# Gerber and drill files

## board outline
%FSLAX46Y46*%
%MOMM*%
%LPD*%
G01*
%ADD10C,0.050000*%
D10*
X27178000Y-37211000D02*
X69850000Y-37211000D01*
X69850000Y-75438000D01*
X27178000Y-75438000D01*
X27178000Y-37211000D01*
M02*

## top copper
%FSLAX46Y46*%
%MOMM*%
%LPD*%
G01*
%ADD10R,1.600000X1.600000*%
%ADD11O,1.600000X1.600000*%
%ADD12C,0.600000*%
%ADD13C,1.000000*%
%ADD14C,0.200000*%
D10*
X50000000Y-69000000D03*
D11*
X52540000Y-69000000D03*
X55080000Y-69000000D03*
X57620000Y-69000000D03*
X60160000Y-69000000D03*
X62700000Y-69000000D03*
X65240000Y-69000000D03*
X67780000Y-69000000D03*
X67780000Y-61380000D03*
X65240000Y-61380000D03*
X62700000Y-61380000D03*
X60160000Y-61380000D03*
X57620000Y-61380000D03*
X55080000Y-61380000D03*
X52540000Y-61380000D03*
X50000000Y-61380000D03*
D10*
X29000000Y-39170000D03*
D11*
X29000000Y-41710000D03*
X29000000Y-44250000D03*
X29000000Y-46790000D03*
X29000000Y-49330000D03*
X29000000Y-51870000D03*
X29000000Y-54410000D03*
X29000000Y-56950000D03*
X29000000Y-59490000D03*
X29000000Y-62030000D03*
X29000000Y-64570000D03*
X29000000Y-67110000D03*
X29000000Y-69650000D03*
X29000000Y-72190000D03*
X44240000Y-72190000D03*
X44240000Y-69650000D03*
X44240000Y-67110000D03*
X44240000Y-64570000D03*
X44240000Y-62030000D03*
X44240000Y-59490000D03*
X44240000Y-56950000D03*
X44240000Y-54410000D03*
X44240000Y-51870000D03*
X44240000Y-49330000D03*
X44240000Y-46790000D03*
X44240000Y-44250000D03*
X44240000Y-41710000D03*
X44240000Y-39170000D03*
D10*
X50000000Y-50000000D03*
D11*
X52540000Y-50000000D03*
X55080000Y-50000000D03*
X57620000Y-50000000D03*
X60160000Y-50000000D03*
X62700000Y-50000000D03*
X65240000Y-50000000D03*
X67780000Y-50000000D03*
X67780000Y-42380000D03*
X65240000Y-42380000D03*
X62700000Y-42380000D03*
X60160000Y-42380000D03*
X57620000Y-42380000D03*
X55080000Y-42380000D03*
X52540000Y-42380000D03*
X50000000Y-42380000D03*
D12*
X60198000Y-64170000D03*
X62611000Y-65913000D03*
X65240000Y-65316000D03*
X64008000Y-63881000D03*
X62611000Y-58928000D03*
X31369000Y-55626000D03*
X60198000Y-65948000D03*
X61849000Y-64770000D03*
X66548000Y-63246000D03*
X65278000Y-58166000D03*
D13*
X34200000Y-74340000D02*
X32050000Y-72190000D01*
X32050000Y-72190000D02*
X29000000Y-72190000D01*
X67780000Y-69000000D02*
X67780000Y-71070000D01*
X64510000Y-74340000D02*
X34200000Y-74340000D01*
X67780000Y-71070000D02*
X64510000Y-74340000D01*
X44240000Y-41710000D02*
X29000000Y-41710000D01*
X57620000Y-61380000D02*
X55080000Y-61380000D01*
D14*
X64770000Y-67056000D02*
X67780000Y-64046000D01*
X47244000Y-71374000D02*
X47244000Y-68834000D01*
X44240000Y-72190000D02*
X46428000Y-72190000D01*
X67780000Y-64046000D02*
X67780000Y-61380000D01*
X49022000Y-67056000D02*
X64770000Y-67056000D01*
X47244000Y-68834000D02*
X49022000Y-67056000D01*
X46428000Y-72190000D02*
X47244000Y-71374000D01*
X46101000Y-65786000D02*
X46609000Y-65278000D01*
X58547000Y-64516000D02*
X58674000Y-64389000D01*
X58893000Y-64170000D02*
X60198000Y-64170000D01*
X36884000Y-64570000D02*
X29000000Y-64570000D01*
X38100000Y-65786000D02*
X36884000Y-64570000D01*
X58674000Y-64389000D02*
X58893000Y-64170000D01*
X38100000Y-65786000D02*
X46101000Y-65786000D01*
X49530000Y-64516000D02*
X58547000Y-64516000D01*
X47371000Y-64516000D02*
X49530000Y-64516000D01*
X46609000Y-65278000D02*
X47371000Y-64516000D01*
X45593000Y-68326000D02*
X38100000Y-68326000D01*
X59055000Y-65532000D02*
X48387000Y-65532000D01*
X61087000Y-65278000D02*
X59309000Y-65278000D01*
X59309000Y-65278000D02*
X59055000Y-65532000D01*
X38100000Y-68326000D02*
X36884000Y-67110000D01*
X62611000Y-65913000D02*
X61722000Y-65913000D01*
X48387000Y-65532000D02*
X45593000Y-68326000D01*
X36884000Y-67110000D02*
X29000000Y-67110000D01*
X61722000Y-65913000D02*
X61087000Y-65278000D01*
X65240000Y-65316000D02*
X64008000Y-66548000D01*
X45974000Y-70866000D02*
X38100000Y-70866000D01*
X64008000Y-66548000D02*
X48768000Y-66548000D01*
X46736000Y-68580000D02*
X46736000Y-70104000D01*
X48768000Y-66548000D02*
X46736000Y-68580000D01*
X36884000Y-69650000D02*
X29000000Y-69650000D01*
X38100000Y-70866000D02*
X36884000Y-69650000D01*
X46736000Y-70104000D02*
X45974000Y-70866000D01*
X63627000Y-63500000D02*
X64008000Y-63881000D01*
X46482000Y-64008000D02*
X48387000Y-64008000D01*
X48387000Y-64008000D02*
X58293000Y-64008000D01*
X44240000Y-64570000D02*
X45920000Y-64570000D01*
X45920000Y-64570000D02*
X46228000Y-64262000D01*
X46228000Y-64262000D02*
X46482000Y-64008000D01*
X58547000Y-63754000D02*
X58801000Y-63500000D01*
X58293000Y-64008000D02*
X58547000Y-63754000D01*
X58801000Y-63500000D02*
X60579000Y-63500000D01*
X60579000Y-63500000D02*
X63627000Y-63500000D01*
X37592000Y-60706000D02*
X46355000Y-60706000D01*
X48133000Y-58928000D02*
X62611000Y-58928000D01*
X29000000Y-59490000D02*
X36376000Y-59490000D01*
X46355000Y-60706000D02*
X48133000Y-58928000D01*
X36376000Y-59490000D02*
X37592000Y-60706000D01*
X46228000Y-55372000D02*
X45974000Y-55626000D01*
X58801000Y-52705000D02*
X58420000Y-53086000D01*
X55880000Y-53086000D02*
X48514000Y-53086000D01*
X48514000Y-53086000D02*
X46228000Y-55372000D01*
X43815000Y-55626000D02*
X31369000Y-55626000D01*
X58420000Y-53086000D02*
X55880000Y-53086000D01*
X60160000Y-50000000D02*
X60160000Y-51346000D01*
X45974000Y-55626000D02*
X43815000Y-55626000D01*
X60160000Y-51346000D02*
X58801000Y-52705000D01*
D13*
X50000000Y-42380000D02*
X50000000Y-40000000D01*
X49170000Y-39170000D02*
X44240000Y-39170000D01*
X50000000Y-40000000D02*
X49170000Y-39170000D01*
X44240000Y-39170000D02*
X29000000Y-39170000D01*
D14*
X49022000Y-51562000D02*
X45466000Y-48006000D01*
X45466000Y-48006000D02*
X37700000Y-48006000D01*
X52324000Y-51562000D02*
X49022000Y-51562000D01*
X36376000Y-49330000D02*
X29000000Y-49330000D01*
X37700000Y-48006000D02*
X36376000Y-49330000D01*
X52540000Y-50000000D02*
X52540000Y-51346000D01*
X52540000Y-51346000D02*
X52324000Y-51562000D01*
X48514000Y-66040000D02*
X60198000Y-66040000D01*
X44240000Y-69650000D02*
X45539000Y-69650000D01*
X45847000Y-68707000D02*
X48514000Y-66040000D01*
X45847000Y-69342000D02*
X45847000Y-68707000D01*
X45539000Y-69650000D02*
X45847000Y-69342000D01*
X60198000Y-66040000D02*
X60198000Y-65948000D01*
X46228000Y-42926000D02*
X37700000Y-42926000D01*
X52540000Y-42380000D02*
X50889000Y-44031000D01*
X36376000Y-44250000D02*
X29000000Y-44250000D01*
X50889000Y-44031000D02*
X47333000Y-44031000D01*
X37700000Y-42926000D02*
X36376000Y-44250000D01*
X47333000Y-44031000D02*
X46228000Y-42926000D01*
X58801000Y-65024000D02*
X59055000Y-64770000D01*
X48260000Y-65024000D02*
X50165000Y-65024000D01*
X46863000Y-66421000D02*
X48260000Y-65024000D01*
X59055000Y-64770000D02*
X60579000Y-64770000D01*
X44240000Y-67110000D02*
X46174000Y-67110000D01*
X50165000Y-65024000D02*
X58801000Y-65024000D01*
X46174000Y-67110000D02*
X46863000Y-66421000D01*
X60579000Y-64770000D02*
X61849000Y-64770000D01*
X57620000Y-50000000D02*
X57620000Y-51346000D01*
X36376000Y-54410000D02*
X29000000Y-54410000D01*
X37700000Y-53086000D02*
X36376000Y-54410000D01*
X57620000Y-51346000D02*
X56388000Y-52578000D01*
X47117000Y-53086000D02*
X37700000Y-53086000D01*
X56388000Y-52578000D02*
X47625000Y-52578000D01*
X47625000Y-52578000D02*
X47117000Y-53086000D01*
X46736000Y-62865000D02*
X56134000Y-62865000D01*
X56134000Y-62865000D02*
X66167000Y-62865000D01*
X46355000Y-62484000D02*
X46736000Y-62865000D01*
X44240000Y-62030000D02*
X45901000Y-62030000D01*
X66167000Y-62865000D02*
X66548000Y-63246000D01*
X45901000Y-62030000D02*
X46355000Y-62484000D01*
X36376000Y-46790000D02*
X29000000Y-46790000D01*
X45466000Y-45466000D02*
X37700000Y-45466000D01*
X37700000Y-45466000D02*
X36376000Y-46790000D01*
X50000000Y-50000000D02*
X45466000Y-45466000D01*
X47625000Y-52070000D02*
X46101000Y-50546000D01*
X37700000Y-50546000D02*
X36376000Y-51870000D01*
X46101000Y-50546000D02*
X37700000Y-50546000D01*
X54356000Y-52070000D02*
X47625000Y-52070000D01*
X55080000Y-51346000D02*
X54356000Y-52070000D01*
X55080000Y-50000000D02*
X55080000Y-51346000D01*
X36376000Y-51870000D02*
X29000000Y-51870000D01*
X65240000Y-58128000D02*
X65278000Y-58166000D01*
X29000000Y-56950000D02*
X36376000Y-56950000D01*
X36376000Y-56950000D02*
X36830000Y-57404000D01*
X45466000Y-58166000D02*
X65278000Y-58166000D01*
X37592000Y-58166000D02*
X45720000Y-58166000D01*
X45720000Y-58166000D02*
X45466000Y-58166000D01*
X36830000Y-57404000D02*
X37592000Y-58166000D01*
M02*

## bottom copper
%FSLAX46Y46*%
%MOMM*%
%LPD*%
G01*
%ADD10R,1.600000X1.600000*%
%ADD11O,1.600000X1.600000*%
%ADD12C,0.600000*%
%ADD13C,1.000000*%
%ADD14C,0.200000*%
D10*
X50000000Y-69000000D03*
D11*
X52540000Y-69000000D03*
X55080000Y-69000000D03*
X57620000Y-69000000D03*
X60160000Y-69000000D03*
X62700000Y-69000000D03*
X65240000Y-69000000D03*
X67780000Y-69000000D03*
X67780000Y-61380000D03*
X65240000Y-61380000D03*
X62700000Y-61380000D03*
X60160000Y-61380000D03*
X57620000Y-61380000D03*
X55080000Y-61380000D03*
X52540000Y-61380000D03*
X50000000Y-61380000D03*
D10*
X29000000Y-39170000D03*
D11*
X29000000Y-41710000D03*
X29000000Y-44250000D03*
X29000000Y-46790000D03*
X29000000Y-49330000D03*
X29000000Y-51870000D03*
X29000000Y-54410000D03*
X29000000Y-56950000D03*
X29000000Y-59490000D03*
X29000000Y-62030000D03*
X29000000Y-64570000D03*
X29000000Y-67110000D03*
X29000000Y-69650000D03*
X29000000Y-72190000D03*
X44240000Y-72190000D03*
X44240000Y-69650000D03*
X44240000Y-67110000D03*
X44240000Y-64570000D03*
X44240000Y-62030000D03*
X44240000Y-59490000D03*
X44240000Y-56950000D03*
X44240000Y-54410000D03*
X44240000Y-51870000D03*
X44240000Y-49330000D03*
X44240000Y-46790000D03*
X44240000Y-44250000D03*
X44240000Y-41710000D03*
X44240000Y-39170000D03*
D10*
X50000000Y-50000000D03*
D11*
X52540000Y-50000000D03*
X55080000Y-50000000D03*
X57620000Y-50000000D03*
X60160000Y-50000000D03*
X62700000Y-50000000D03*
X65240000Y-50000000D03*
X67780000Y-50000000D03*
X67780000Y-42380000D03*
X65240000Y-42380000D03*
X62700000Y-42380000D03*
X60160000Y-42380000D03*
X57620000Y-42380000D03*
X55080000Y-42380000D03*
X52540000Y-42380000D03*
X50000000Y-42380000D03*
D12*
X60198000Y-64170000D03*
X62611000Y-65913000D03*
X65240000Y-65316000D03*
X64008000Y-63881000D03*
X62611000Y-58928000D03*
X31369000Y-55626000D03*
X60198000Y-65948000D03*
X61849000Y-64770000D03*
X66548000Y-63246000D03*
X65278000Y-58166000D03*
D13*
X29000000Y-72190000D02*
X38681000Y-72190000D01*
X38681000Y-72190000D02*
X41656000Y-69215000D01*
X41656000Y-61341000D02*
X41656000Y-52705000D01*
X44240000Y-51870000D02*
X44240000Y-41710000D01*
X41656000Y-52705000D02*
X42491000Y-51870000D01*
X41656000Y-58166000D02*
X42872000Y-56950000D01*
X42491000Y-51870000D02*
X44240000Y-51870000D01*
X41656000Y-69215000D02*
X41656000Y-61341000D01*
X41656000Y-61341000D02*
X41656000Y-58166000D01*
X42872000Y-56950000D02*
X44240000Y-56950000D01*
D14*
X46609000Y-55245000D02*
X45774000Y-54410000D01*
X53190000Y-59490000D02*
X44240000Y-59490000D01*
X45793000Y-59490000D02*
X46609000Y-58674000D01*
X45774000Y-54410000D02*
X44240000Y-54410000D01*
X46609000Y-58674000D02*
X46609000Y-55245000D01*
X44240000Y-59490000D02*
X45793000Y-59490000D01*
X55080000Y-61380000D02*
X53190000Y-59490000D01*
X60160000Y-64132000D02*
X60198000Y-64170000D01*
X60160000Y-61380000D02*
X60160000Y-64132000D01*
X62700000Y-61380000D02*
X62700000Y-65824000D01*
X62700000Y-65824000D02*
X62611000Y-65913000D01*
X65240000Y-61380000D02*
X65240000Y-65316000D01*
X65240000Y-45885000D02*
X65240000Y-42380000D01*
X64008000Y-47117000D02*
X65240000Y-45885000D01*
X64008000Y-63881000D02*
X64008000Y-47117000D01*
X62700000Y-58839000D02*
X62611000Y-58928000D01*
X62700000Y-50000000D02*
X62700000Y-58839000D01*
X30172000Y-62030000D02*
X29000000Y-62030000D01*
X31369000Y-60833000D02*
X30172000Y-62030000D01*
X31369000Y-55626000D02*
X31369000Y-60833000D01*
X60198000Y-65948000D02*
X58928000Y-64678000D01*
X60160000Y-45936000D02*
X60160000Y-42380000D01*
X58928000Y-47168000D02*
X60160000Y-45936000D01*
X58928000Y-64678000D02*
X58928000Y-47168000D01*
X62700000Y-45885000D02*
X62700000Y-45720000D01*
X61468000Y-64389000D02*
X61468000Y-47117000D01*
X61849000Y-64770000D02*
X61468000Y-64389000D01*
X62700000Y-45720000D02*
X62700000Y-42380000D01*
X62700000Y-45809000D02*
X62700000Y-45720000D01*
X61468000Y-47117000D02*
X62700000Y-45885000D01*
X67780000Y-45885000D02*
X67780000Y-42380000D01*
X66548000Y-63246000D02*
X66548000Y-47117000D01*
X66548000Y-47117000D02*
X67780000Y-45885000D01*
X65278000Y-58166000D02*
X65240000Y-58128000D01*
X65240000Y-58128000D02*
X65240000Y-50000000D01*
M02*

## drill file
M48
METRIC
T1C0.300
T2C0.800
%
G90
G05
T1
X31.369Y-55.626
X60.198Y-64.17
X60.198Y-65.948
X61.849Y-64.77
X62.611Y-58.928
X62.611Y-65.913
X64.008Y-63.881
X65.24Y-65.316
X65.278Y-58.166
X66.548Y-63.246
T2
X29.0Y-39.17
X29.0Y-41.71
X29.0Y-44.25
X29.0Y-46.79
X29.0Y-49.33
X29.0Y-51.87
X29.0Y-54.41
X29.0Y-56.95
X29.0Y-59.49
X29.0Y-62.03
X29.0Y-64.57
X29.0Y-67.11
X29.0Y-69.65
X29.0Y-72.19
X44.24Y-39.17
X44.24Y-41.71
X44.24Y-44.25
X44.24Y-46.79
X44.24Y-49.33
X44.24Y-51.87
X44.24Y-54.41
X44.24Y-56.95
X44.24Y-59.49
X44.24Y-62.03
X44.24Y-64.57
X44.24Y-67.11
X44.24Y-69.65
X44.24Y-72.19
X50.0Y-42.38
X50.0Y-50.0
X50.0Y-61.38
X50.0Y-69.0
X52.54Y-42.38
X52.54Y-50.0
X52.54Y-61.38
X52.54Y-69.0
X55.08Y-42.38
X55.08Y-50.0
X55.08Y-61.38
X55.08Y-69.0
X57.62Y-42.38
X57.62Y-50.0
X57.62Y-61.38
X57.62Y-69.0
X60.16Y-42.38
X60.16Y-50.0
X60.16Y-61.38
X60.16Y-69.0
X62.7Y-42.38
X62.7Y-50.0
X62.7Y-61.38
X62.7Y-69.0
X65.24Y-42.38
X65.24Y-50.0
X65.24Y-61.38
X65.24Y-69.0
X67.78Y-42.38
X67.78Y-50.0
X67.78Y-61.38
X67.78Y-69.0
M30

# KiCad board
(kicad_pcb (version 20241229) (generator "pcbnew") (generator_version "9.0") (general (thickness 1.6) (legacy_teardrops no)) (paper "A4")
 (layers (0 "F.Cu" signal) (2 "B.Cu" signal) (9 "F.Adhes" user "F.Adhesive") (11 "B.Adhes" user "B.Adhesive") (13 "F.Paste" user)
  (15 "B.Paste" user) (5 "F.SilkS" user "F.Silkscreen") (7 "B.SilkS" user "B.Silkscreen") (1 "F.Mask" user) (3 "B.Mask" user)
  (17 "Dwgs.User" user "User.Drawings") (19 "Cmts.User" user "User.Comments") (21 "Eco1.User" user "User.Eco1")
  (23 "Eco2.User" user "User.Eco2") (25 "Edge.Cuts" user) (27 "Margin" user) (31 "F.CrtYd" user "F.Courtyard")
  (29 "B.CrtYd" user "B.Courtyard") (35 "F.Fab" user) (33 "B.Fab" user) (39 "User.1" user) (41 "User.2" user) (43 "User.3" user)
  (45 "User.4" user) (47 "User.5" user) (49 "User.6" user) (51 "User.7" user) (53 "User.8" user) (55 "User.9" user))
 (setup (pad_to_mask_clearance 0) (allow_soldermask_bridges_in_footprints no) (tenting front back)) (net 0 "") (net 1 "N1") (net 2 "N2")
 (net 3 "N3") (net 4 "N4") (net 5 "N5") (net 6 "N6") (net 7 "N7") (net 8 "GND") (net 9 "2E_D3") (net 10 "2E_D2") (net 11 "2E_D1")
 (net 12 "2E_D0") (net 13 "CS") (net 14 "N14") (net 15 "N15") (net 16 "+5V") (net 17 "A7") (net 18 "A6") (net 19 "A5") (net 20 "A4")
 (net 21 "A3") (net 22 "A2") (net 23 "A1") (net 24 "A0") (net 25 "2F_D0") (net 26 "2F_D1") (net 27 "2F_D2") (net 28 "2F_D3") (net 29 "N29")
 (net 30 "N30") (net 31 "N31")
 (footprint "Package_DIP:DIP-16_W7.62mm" (layer "F.Cu") (at 50 69 90)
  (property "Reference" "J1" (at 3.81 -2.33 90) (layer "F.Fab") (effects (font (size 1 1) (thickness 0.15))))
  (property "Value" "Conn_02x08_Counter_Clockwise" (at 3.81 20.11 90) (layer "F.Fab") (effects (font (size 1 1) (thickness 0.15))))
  (pad "1" thru_hole rect (at 0 0 90) (size 1.6 1.6) (drill 0.8) (layers "*.Cu" "*.Mask") (remove_unused_layers no) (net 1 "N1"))
  (pad "2" thru_hole oval (at 0 2.54 90) (size 1.6 1.6) (drill 0.8) (layers "*.Cu" "*.Mask") (remove_unused_layers no) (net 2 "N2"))
  (pad "3" thru_hole oval (at 0 5.08 90) (size 1.6 1.6) (drill 0.8) (layers "*.Cu" "*.Mask") (remove_unused_layers no) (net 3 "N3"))
  (pad "4" thru_hole oval (at 0 7.62 90) (size 1.6 1.6) (drill 0.8) (layers "*.Cu" "*.Mask") (remove_unused_layers no) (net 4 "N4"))
  (pad "5" thru_hole oval (at 0 10.16 90) (size 1.6 1.6) (drill 0.8) (layers "*.Cu" "*.Mask") (remove_unused_layers no) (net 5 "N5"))
  (pad "6" thru_hole oval (at 0 12.7 90) (size 1.6 1.6) (drill 0.8) (layers "*.Cu" "*.Mask") (remove_unused_layers no) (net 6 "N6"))
  (pad "7" thru_hole oval (at 0 15.24 90) (size 1.6 1.6) (drill 0.8) (layers "*.Cu" "*.Mask") (remove_unused_layers no) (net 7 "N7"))
  (pad "8" thru_hole oval (at 0 17.78 90) (size 1.6 1.6) (drill 0.8) (layers "*.Cu" "*.Mask") (remove_unused_layers no) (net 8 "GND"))
  (pad "9" thru_hole oval (at 7.62 17.78 90) (size 1.6 1.6) (drill 0.8) (layers "*.Cu" "*.Mask") (remove_unused_layers no) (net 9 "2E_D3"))
  (pad "10" thru_hole oval (at 7.62 15.24 90) (size 1.6 1.6) (drill 0.8) (layers "*.Cu" "*.Mask") (remove_unused_layers no) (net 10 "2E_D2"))
  (pad "11" thru_hole oval (at 7.62 12.7 90) (size 1.6 1.6) (drill 0.8) (layers "*.Cu" "*.Mask") (remove_unused_layers no) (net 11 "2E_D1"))
  (pad "12" thru_hole oval (at 7.62 10.16 90) (size 1.6 1.6) (drill 0.8) (layers "*.Cu" "*.Mask") (remove_unused_layers no) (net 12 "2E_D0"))
  (pad "13" thru_hole oval (at 7.62 7.62 90) (size 1.6 1.6) (drill 0.8) (layers "*.Cu" "*.Mask") (remove_unused_layers no) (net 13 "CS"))
  (pad "14" thru_hole oval (at 7.62 5.08 90) (size 1.6 1.6) (drill 0.8) (layers "*.Cu" "*.Mask") (remove_unused_layers no) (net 13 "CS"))
  (pad "15" thru_hole oval (at 7.62 2.54 90) (size 1.6 1.6) (drill 0.8) (layers "*.Cu" "*.Mask") (remove_unused_layers no) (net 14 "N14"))
  (pad "16" thru_hole oval (at 7.62 0 90) (size 1.6 1.6) (drill 0.8) (layers "*.Cu" "*.Mask") (remove_unused_layers no) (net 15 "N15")))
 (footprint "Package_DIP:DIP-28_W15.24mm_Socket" (layer "F.Cu") (at 29 39.17)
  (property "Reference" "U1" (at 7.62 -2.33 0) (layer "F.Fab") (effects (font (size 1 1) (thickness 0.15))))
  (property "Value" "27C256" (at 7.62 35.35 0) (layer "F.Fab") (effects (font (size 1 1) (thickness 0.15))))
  (pad "1" thru_hole rect (at 0 0) (size 1.6 1.6) (drill 0.8) (layers "*.Cu" "*.Mask") (remove_unused_layers no) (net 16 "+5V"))
  (pad "2" thru_hole oval (at 0 2.54) (size 1.6 1.6) (drill 0.8) (layers "*.Cu" "*.Mask") (remove_unused_layers no) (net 8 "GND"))
  (pad "3" thru_hole oval (at 0 5.08) (size 1.6 1.6) (drill 0.8) (layers "*.Cu" "*.Mask") (remove_unused_layers no) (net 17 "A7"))
  (pad "4" thru_hole oval (at 0 7.62) (size 1.6 1.6) (drill 0.8) (layers "*.Cu" "*.Mask") (remove_unused_layers no) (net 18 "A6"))
  (pad "5" thru_hole oval (at 0 10.16) (size 1.6 1.6) (drill 0.8) (layers "*.Cu" "*.Mask") (remove_unused_layers no) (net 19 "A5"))
  (pad "6" thru_hole oval (at 0 12.7) (size 1.6 1.6) (drill 0.8) (layers "*.Cu" "*.Mask") (remove_unused_layers no) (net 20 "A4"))
  (pad "7" thru_hole oval (at 0 15.24) (size 1.6 1.6) (drill 0.8) (layers "*.Cu" "*.Mask") (remove_unused_layers no) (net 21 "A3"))
  (pad "8" thru_hole oval (at 0 17.78) (size 1.6 1.6) (drill 0.8) (layers "*.Cu" "*.Mask") (remove_unused_layers no) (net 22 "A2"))
  (pad "9" thru_hole oval (at 0 20.32) (size 1.6 1.6) (drill 0.8) (layers "*.Cu" "*.Mask") (remove_unused_layers no) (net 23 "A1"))
  (pad "10" thru_hole oval (at 0 22.86) (size 1.6 1.6) (drill 0.8) (layers "*.Cu" "*.Mask") (remove_unused_layers no) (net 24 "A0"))
  (pad "11" thru_hole oval (at 0 25.4) (size 1.6 1.6) (drill 0.8) (layers "*.Cu" "*.Mask") (remove_unused_layers no) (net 12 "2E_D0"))
  (pad "12" thru_hole oval (at 0 27.94) (size 1.6 1.6) (drill 0.8) (layers "*.Cu" "*.Mask") (remove_unused_layers no) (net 11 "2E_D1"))
  (pad "13" thru_hole oval (at 0 30.48) (size 1.6 1.6) (drill 0.8) (layers "*.Cu" "*.Mask") (remove_unused_layers no) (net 10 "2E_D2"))
  (pad "14" thru_hole oval (at 0 33.02) (size 1.6 1.6) (drill 0.8) (layers "*.Cu" "*.Mask") (remove_unused_layers no) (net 8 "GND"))
  (pad "15" thru_hole oval (at 15.24 33.02) (size 1.6 1.6) (drill 0.8) (layers "*.Cu" "*.Mask") (remove_unused_layers no) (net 9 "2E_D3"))
  (pad "16" thru_hole oval (at 15.24 30.48) (size 1.6 1.6) (drill 0.8) (layers "*.Cu" "*.Mask") (remove_unused_layers no) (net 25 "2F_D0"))
  (pad "17" thru_hole oval (at 15.24 27.94) (size 1.6 1.6) (drill 0.8) (layers "*.Cu" "*.Mask") (remove_unused_layers no) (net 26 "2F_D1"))
  (pad "18" thru_hole oval (at 15.24 25.4) (size 1.6 1.6) (drill 0.8) (layers "*.Cu" "*.Mask") (remove_unused_layers no) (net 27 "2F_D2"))
  (pad "19" thru_hole oval (at 15.24 22.86) (size 1.6 1.6) (drill 0.8) (layers "*.Cu" "*.Mask") (remove_unused_layers no) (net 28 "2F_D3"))
  (pad "20" thru_hole oval (at 15.24 20.32) (size 1.6 1.6) (drill 0.8) (layers "*.Cu" "*.Mask") (remove_unused_layers no) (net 13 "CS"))
  (pad "21" thru_hole oval (at 15.24 17.78) (size 1.6 1.6) (drill 0.8) (layers "*.Cu" "*.Mask") (remove_unused_layers no) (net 8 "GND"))
  (pad "22" thru_hole oval (at 15.24 15.24) (size 1.6 1.6) (drill 0.8) (layers "*.Cu" "*.Mask") (remove_unused_layers no) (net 13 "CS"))
  (pad "23" thru_hole oval (at 15.24 12.7) (size 1.6 1.6) (drill 0.8) (layers "*.Cu" "*.Mask") (remove_unused_layers no) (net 8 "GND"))
  (pad "24" thru_hole oval (at 15.24 10.16) (size 1.6 1.6) (drill 0.8) (layers "*.Cu" "*.Mask") (remove_unused_layers no) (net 8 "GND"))
  (pad "25" thru_hole oval (at 15.24 7.62) (size 1.6 1.6) (drill 0.8) (layers "*.Cu" "*.Mask") (remove_unused_layers no) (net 8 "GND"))
  (pad "26" thru_hole oval (at 15.24 5.08) (size 1.6 1.6) (drill 0.8) (layers "*.Cu" "*.Mask") (remove_unused_layers no) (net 8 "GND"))
  (pad "27" thru_hole oval (at 15.24 2.54) (size 1.6 1.6) (drill 0.8) (layers "*.Cu" "*.Mask") (remove_unused_layers no) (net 8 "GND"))
  (pad "28" thru_hole oval (at 15.24 0) (size 1.6 1.6) (drill 0.8) (layers "*.Cu" "*.Mask") (remove_unused_layers no) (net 16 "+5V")))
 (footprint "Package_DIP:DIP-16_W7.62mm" (layer "F.Cu") (at 50 50 90)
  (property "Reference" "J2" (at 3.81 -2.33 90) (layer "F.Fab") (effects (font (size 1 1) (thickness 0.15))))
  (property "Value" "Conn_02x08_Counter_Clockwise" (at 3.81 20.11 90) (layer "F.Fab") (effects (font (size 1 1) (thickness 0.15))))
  (pad "1" thru_hole rect (at 0 0 90) (size 1.6 1.6) (drill 0.8) (layers "*.Cu" "*.Mask") (remove_unused_layers no) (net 18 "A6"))
  (pad "2" thru_hole oval (at 0 2.54 90) (size 1.6 1.6) (drill 0.8) (layers "*.Cu" "*.Mask") (remove_unused_layers no) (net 19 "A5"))
  (pad "3" thru_hole oval (at 0 5.08 90) (size 1.6 1.6) (drill 0.8) (layers "*.Cu" "*.Mask") (remove_unused_layers no) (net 20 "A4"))
  (pad "4" thru_hole oval (at 0 7.62 90) (size 1.6 1.6) (drill 0.8) (layers "*.Cu" "*.Mask") (remove_unused_layers no) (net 21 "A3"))
  (pad "5" thru_hole oval (at 0 10.16 90) (size 1.6 1.6) (drill 0.8) (layers "*.Cu" "*.Mask") (remove_unused_layers no) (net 24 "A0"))
  (pad "6" thru_hole oval (at 0 12.7 90) (size 1.6 1.6) (drill 0.8) (layers "*.Cu" "*.Mask") (remove_unused_layers no) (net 23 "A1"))
  (pad "7" thru_hole oval (at 0 15.24 90) (size 1.6 1.6) (drill 0.8) (layers "*.Cu" "*.Mask") (remove_unused_layers no) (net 22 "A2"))
  (pad "8" thru_hole oval (at 0 17.78 90) (size 1.6 1.6) (drill 0.8) (layers "*.Cu" "*.Mask") (remove_unused_layers no) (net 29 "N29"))
  (pad "9" thru_hole oval (at 7.62 17.78 90) (size 1.6 1.6) (drill 0.8) (layers "*.Cu" "*.Mask") (remove_unused_layers no) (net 28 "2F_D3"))
  (pad "10" thru_hole oval (at 7.62 15.24 90) (size 1.6 1.6) (drill 0.8) (layers "*.Cu" "*.Mask") (remove_unused_layers no) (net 27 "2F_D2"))
  (pad "11" thru_hole oval (at 7.62 12.7 90) (size 1.6 1.6) (drill 0.8) (layers "*.Cu" "*.Mask") (remove_unused_layers no) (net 26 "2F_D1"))
  (pad "12" thru_hole oval (at 7.62 10.16 90) (size 1.6 1.6) (drill 0.8) (layers "*.Cu" "*.Mask") (remove_unused_layers no) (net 25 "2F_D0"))
  (pad "13" thru_hole oval (at 7.62 7.62 90) (size 1.6 1.6) (drill 0.8) (layers "*.Cu" "*.Mask") (remove_unused_layers no) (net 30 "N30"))
  (pad "14" thru_hole oval (at 7.62 5.08 90) (size 1.6 1.6) (drill 0.8) (layers "*.Cu" "*.Mask") (remove_unused_layers no) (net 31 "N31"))
  (pad "15" thru_hole oval (at 7.62 2.54 90) (size 1.6 1.6) (drill 0.8) (layers "*.Cu" "*.Mask") (remove_unused_layers no) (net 17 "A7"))
  (pad "16" thru_hole oval (at 7.62 0 90) (size 1.6 1.6) (drill 0.8) (layers "*.Cu" "*.Mask") (remove_unused_layers no) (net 16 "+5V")))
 (gr_rect (start 27.178 37.211) (end 69.85 75.438) (stroke (width 0.05) (type default)) (fill no) (layer "Edge.Cuts"))
 (segment (start 34.2 74.34) (end 32.05 72.19) (width 1) (layer "F.Cu") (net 8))
 (segment (start 32.05 72.19) (end 29 72.19) (width 1) (layer "F.Cu") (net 8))
 (segment (start 67.78 69) (end 67.78 71.07) (width 1) (layer "F.Cu") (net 8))
 (segment (start 64.51 74.34) (end 34.2 74.34) (width 1) (layer "F.Cu") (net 8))
 (segment (start 67.78 71.07) (end 64.51 74.34) (width 1) (layer "F.Cu") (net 8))
 (segment (start 44.24 41.71) (end 29 41.71) (width 1) (layer "F.Cu") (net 8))
 (segment (start 29 72.19) (end 38.681 72.19) (width 1) (layer "B.Cu") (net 8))
 (segment (start 38.681 72.19) (end 41.656 69.215) (width 1) (layer "B.Cu") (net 8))
 (segment (start 41.656 61.341) (end 41.656 52.705) (width 1) (layer "B.Cu") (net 8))
 (segment (start 44.24 51.87) (end 44.24 41.71) (width 1) (layer "B.Cu") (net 8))
 (segment (start 41.656 52.705) (end 42.491 51.87) (width 1) (layer "B.Cu") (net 8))
 (segment (start 41.656 58.166) (end 42.872 56.95) (width 1) (layer "B.Cu") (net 8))
 (segment (start 42.491 51.87) (end 44.24 51.87) (width 1) (layer "B.Cu") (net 8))
 (segment (start 41.656 69.215) (end 41.656 61.341) (width 1) (layer "B.Cu") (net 8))
 (segment (start 41.656 61.341) (end 41.656 58.166) (width 1) (layer "B.Cu") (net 8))
 (segment (start 42.872 56.95) (end 44.24 56.95) (width 1) (layer "B.Cu") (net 8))
 (segment (start 57.62 61.38) (end 55.08 61.38) (width 1) (layer "F.Cu") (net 13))
 (segment (start 46.609 55.245) (end 45.774 54.41) (width 0.2) (layer "B.Cu") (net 13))
 (segment (start 53.19 59.49) (end 44.24 59.49) (width 0.2) (layer "B.Cu") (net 13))
 (segment (start 45.793 59.49) (end 46.609 58.674) (width 0.2) (layer "B.Cu") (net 13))
 (segment (start 45.774 54.41) (end 44.24 54.41) (width 0.2) (layer "B.Cu") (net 13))
 (segment (start 46.609 58.674) (end 46.609 55.245) (width 0.2) (layer "B.Cu") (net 13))
 (segment (start 44.24 59.49) (end 45.793 59.49) (width 0.2) (layer "B.Cu") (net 13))
 (segment (start 55.08 61.38) (end 53.19 59.49) (width 0.2) (layer "B.Cu") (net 13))
 (segment (start 64.77 67.056) (end 67.78 64.046) (width 0.2) (layer "F.Cu") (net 9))
 (segment (start 47.244 71.374) (end 47.244 68.834) (width 0.2) (layer "F.Cu") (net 9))
 (segment (start 44.24 72.19) (end 46.428 72.19) (width 0.2) (layer "F.Cu") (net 9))
 (segment (start 67.78 64.046) (end 67.78 61.38) (width 0.2) (layer "F.Cu") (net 9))
 (segment (start 49.022 67.056) (end 64.77 67.056) (width 0.2) (layer "F.Cu") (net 9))
 (segment (start 47.244 68.834) (end 49.022 67.056) (width 0.2) (layer "F.Cu") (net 9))
 (segment (start 46.428 72.19) (end 47.244 71.374) (width 0.2) (layer "F.Cu") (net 9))
 (segment (start 46.101 65.786) (end 46.609 65.278) (width 0.2) (layer "F.Cu") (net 12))
 (segment (start 58.547 64.516) (end 58.674 64.389) (width 0.2) (layer "F.Cu") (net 12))
 (segment (start 58.893 64.17) (end 60.198 64.17) (width 0.2) (layer "F.Cu") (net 12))
 (segment (start 36.884 64.57) (end 29 64.57) (width 0.2) (layer "F.Cu") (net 12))
 (segment (start 38.1 65.786) (end 36.884 64.57) (width 0.2) (layer "F.Cu") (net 12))
 (segment (start 58.674 64.389) (end 58.893 64.17) (width 0.2) (layer "F.Cu") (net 12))
 (segment (start 38.1 65.786) (end 46.101 65.786) (width 0.2) (layer "F.Cu") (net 12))
 (segment (start 49.53 64.516) (end 58.547 64.516) (width 0.2) (layer "F.Cu") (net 12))
 (segment (start 47.371 64.516) (end 49.53 64.516) (width 0.2) (layer "F.Cu") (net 12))
 (segment (start 46.609 65.278) (end 47.371 64.516) (width 0.2) (layer "F.Cu") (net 12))
 (via (at 60.198 64.17) (size 0.6) (drill 0.3) (layers "F.Cu" "B.Cu") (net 12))
 (segment (start 60.16 64.132) (end 60.198 64.17) (width 0.2) (layer "B.Cu") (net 12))
 (segment (start 60.16 61.38) (end 60.16 64.132) (width 0.2) (layer "B.Cu") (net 12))
 (segment (start 45.593 68.326) (end 38.1 68.326) (width 0.2) (layer "F.Cu") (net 11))
 (segment (start 59.055 65.532) (end 48.387 65.532) (width 0.2) (layer "F.Cu") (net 11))
 (segment (start 61.087 65.278) (end 59.309 65.278) (width 0.2) (layer "F.Cu") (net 11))
 (segment (start 59.309 65.278) (end 59.055 65.532) (width 0.2) (layer "F.Cu") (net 11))
 (segment (start 38.1 68.326) (end 36.884 67.11) (width 0.2) (layer "F.Cu") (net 11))
 (segment (start 62.611 65.913) (end 61.722 65.913) (width 0.2) (layer "F.Cu") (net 11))
 (segment (start 48.387 65.532) (end 45.593 68.326) (width 0.2) (layer "F.Cu") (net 11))
 (segment (start 36.884 67.11) (end 29 67.11) (width 0.2) (layer "F.Cu") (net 11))
 (segment (start 61.722 65.913) (end 61.087 65.278) (width 0.2) (layer "F.Cu") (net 11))
 (via (at 62.611 65.913) (size 0.6) (drill 0.3) (layers "F.Cu" "B.Cu") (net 11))
 (segment (start 62.7 61.38) (end 62.7 65.824) (width 0.2) (layer "B.Cu") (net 11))
 (segment (start 62.7 65.824) (end 62.611 65.913) (width 0.2) (layer "B.Cu") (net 11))
 (segment (start 65.24 65.316) (end 64.008 66.548) (width 0.2) (layer "F.Cu") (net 10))
 (segment (start 45.974 70.866) (end 38.1 70.866) (width 0.2) (layer "F.Cu") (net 10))
 (segment (start 64.008 66.548) (end 48.768 66.548) (width 0.2) (layer "F.Cu") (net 10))
 (segment (start 46.736 68.58) (end 46.736 70.104) (width 0.2) (layer "F.Cu") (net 10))
 (segment (start 48.768 66.548) (end 46.736 68.58) (width 0.2) (layer "F.Cu") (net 10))
 (segment (start 36.884 69.65) (end 29 69.65) (width 0.2) (layer "F.Cu") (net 10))
 (segment (start 38.1 70.866) (end 36.884 69.65) (width 0.2) (layer "F.Cu") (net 10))
 (segment (start 46.736 70.104) (end 45.974 70.866) (width 0.2) (layer "F.Cu") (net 10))
 (via (at 65.24 65.316) (size 0.6) (drill 0.3) (layers "F.Cu" "B.Cu") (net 10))
 (segment (start 65.24 61.38) (end 65.24 65.316) (width 0.2) (layer "B.Cu") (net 10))
 (segment (start 63.627 63.5) (end 64.008 63.881) (width 0.2) (layer "F.Cu") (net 27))
 (segment (start 46.482 64.008) (end 48.387 64.008) (width 0.2) (layer "F.Cu") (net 27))
 (segment (start 48.387 64.008) (end 58.293 64.008) (width 0.2) (layer "F.Cu") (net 27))
 (segment (start 44.24 64.57) (end 45.92 64.57) (width 0.2) (layer "F.Cu") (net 27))
 (segment (start 45.92 64.57) (end 46.228 64.262) (width 0.2) (layer "F.Cu") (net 27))
 (segment (start 46.228 64.262) (end 46.482 64.008) (width 0.2) (layer "F.Cu") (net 27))
 (segment (start 58.547 63.754) (end 58.801 63.5) (width 0.2) (layer "F.Cu") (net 27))
 (segment (start 58.293 64.008) (end 58.547 63.754) (width 0.2) (layer "F.Cu") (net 27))
 (segment (start 58.801 63.5) (end 60.579 63.5) (width 0.2) (layer "F.Cu") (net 27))
 (segment (start 60.579 63.5) (end 63.627 63.5) (width 0.2) (layer "F.Cu") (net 27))
 (via (at 64.008 63.881) (size 0.6) (drill 0.3) (layers "F.Cu" "B.Cu") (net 27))
 (segment (start 65.24 45.885) (end 65.24 42.38) (width 0.2) (layer "B.Cu") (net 27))
 (segment (start 64.008 47.117) (end 65.24 45.885) (width 0.2) (layer "B.Cu") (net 27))
 (segment (start 64.008 63.881) (end 64.008 47.117) (width 0.2) (layer "B.Cu") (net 27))
 (segment (start 37.592 60.706) (end 46.355 60.706) (width 0.2) (layer "F.Cu") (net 23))
 (segment (start 48.133 58.928) (end 62.611 58.928) (width 0.2) (layer "F.Cu") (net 23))
 (segment (start 29 59.49) (end 36.376 59.49) (width 0.2) (layer "F.Cu") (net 23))
 (segment (start 46.355 60.706) (end 48.133 58.928) (width 0.2) (layer "F.Cu") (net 23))
 (segment (start 36.376 59.49) (end 37.592 60.706) (width 0.2) (layer "F.Cu") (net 23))
 (via (at 62.611 58.928) (size 0.6) (drill 0.3) (layers "F.Cu" "B.Cu") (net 23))
 (segment (start 62.7 58.839) (end 62.611 58.928) (width 0.2) (layer "B.Cu") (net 23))
 (segment (start 62.7 50) (end 62.7 58.839) (width 0.2) (layer "B.Cu") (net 23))
 (segment (start 46.228 55.372) (end 45.974 55.626) (width 0.2) (layer "F.Cu") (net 24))
 (segment (start 58.801 52.705) (end 58.42 53.086) (width 0.2) (layer "F.Cu") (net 24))
 (segment (start 55.88 53.086) (end 48.514 53.086) (width 0.2) (layer "F.Cu") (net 24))
 (segment (start 48.514 53.086) (end 46.228 55.372) (width 0.2) (layer "F.Cu") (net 24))
 (segment (start 43.815 55.626) (end 31.369 55.626) (width 0.2) (layer "F.Cu") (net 24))
 (segment (start 58.42 53.086) (end 55.88 53.086) (width 0.2) (layer "F.Cu") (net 24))
 (segment (start 60.16 50) (end 60.16 51.346) (width 0.2) (layer "F.Cu") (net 24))
 (segment (start 45.974 55.626) (end 43.815 55.626) (width 0.2) (layer "F.Cu") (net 24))
 (segment (start 60.16 51.346) (end 58.801 52.705) (width 0.2) (layer "F.Cu") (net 24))
 (via (at 31.369 55.626) (size 0.6) (drill 0.3) (layers "F.Cu" "B.Cu") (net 24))
 (segment (start 30.172 62.03) (end 29 62.03) (width 0.2) (layer "B.Cu") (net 24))
 (segment (start 31.369 60.833) (end 30.172 62.03) (width 0.2) (layer "B.Cu") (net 24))
 (segment (start 31.369 55.626) (end 31.369 60.833) (width 0.2) (layer "B.Cu") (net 24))
 (segment (start 50 42.38) (end 50 40) (width 1) (layer "F.Cu") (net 16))
 (segment (start 49.17 39.17) (end 44.24 39.17) (width 1) (layer "F.Cu") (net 16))
 (segment (start 50 40) (end 49.17 39.17) (width 1) (layer "F.Cu") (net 16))
 (segment (start 44.24 39.17) (end 29 39.17) (width 1) (layer "F.Cu") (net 16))
 (segment (start 49.022 51.562) (end 45.466 48.006) (width 0.2) (layer "F.Cu") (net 19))
 (segment (start 45.466 48.006) (end 37.7 48.006) (width 0.2) (layer "F.Cu") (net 19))
 (segment (start 52.324 51.562) (end 49.022 51.562) (width 0.2) (layer "F.Cu") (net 19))
 (segment (start 36.376 49.33) (end 29 49.33) (width 0.2) (layer "F.Cu") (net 19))
 (segment (start 37.7 48.006) (end 36.376 49.33) (width 0.2) (layer "F.Cu") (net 19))
 (segment (start 52.54 50) (end 52.54 51.346) (width 0.2) (layer "F.Cu") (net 19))
 (segment (start 52.54 51.346) (end 52.324 51.562) (width 0.2) (layer "F.Cu") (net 19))
 (segment (start 48.514 66.04) (end 60.198 66.04) (width 0.2) (layer "F.Cu") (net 25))
 (segment (start 44.24 69.65) (end 45.539 69.65) (width 0.2) (layer "F.Cu") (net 25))
 (segment (start 45.847 68.707) (end 48.514 66.04) (width 0.2) (layer "F.Cu") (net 25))
 (segment (start 45.847 69.342) (end 45.847 68.707) (width 0.2) (layer "F.Cu") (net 25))
 (segment (start 45.539 69.65) (end 45.847 69.342) (width 0.2) (layer "F.Cu") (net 25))
 (segment (start 60.198 66.04) (end 60.198 65.948) (width 0.2) (layer "F.Cu") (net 25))
 (via (at 60.198 65.948) (size 0.6) (drill 0.3) (layers "F.Cu" "B.Cu") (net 25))
 (segment (start 60.198 65.948) (end 58.928 64.678) (width 0.2) (layer "B.Cu") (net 25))
 (segment (start 60.16 45.936) (end 60.16 42.38) (width 0.2) (layer "B.Cu") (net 25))
 (segment (start 58.928 47.168) (end 60.16 45.936) (width 0.2) (layer "B.Cu") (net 25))
 (segment (start 58.928 64.678) (end 58.928 47.168) (width 0.2) (layer "B.Cu") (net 25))
 (segment (start 46.228 42.926) (end 37.7 42.926) (width 0.2) (layer "F.Cu") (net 17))
 (segment (start 52.54 42.38) (end 50.889 44.031) (width 0.2) (layer "F.Cu") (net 17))
 (segment (start 36.376 44.25) (end 29 44.25) (width 0.2) (layer "F.Cu") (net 17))
 (segment (start 50.889 44.031) (end 47.333 44.031) (width 0.2) (layer "F.Cu") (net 17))
 (segment (start 37.7 42.926) (end 36.376 44.25) (width 0.2) (layer "F.Cu") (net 17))
 (segment (start 47.333 44.031) (end 46.228 42.926) (width 0.2) (layer "F.Cu") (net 17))
 (segment (start 58.801 65.024) (end 59.055 64.77) (width 0.2) (layer "F.Cu") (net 26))
 (segment (start 48.26 65.024) (end 50.165 65.024) (width 0.2) (layer "F.Cu") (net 26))
 (segment (start 46.863 66.421) (end 48.26 65.024) (width 0.2) (layer "F.Cu") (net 26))
 (segment (start 59.055 64.77) (end 60.579 64.77) (width 0.2) (layer "F.Cu") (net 26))
 (segment (start 44.24 67.11) (end 46.174 67.11) (width 0.2) (layer "F.Cu") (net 26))
 (segment (start 50.165 65.024) (end 58.801 65.024) (width 0.2) (layer "F.Cu") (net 26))
 (segment (start 46.174 67.11) (end 46.863 66.421) (width 0.2) (layer "F.Cu") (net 26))
 (segment (start 60.579 64.77) (end 61.849 64.77) (width 0.2) (layer "F.Cu") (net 26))
 (via (at 61.849 64.77) (size 0.6) (drill 0.3) (layers "F.Cu" "B.Cu") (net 26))
 (segment (start 62.7 45.885) (end 62.7 45.72) (width 0.2) (layer "B.Cu") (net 26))
 (segment (start 61.468 64.389) (end 61.468 47.117) (width 0.2) (layer "B.Cu") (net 26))
 (segment (start 61.849 64.77) (end 61.468 64.389) (width 0.2) (layer "B.Cu") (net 26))
 (segment (start 62.7 45.72) (end 62.7 42.38) (width 0.2) (layer "B.Cu") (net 26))
 (segment (start 62.7 45.809) (end 62.7 45.72) (width 0.2) (layer "B.Cu") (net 26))
 (segment (start 61.468 47.117) (end 62.7 45.885) (width 0.2) (layer "B.Cu") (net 26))
 (segment (start 57.62 50) (end 57.62 51.346) (width 0.2) (layer "F.Cu") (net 21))
 (segment (start 36.376 54.41) (end 29 54.41) (width 0.2) (layer "F.Cu") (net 21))
 (segment (start 37.7 53.086) (end 36.376 54.41) (width 0.2) (layer "F.Cu") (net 21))
 (segment (start 57.62 51.346) (end 56.388 52.578) (width 0.2) (layer "F.Cu") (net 21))
 (segment (start 47.117 53.086) (end 37.7 53.086) (width 0.2) (layer "F.Cu") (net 21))
 (segment (start 56.388 52.578) (end 47.625 52.578) (width 0.2) (layer "F.Cu") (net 21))
 (segment (start 47.625 52.578) (end 47.117 53.086) (width 0.2) (layer "F.Cu") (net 21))
 (segment (start 46.736 62.865) (end 56.134 62.865) (width 0.2) (layer "F.Cu") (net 28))
 (segment (start 56.134 62.865) (end 66.167 62.865) (width 0.2) (layer "F.Cu") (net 28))
 (segment (start 46.355 62.484) (end 46.736 62.865) (width 0.2) (layer "F.Cu") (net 28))
 (segment (start 44.24 62.03) (end 45.901 62.03) (width 0.2) (layer "F.Cu") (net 28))
 (segment (start 66.167 62.865) (end 66.548 63.246) (width 0.2) (layer "F.Cu") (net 28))
 (segment (start 45.901 62.03) (end 46.355 62.484) (width 0.2) (layer "F.Cu") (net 28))
 (via (at 66.548 63.246) (size 0.6) (drill 0.3) (layers "F.Cu" "B.Cu") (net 28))
 (segment (start 67.78 45.885) (end 67.78 42.38) (width 0.2) (layer "B.Cu") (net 28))
 (segment (start 66.548 63.246) (end 66.548 47.117) (width 0.2) (layer "B.Cu") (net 28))
 (segment (start 66.548 47.117) (end 67.78 45.885) (width 0.2) (layer "B.Cu") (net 28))
 (segment (start 36.376 46.79) (end 29 46.79) (width 0.2) (layer "F.Cu") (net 18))
 (segment (start 45.466 45.466) (end 37.7 45.466) (width 0.2) (layer "F.Cu") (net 18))
 (segment (start 37.7 45.466) (end 36.376 46.79) (width 0.2) (layer "F.Cu") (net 18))
 (segment (start 50 50) (end 45.466 45.466) (width 0.2) (layer "F.Cu") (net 18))
 (segment (start 47.625 52.07) (end 46.101 50.546) (width 0.2) (layer "F.Cu") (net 20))
 (segment (start 37.7 50.546) (end 36.376 51.87) (width 0.2) (layer "F.Cu") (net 20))
 (segment (start 46.101 50.546) (end 37.7 50.546) (width 0.2) (layer "F.Cu") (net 20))
 (segment (start 54.356 52.07) (end 47.625 52.07) (width 0.2) (layer "F.Cu") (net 20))
 (segment (start 55.08 51.346) (end 54.356 52.07) (width 0.2) (layer "F.Cu") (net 20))
 (segment (start 55.08 50) (end 55.08 51.346) (width 0.2) (layer "F.Cu") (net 20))
 (segment (start 36.376 51.87) (end 29 51.87) (width 0.2) (layer "F.Cu") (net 20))
 (segment (start 65.24 58.128) (end 65.278 58.166) (width 0.2) (layer "F.Cu") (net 22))
 (segment (start 29 56.95) (end 36.376 56.95) (width 0.2) (layer "F.Cu") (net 22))
 (segment (start 36.376 56.95) (end 36.83 57.404) (width 0.2) (layer "F.Cu") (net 22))
 (segment (start 45.466 58.166) (end 65.278 58.166) (width 0.2) (layer "F.Cu") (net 22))
 (segment (start 37.592 58.166) (end 45.72 58.166) (width 0.2) (layer "F.Cu") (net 22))
 (segment (start 45.72 58.166) (end 45.466 58.166) (width 0.2) (layer "F.Cu") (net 22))
 (segment (start 36.83 57.404) (end 37.592 58.166) (width 0.2) (layer "F.Cu") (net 22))
 (via (at 65.278 58.166) (size 0.6) (drill 0.3) (layers "F.Cu" "B.Cu") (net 22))
 (segment (start 65.278 58.166) (end 65.24 58.128) (width 0.2) (layer "B.Cu") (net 22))
 (segment (start 65.24 58.128) (end 65.24 50) (width 0.2) (layer "B.Cu") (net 22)))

